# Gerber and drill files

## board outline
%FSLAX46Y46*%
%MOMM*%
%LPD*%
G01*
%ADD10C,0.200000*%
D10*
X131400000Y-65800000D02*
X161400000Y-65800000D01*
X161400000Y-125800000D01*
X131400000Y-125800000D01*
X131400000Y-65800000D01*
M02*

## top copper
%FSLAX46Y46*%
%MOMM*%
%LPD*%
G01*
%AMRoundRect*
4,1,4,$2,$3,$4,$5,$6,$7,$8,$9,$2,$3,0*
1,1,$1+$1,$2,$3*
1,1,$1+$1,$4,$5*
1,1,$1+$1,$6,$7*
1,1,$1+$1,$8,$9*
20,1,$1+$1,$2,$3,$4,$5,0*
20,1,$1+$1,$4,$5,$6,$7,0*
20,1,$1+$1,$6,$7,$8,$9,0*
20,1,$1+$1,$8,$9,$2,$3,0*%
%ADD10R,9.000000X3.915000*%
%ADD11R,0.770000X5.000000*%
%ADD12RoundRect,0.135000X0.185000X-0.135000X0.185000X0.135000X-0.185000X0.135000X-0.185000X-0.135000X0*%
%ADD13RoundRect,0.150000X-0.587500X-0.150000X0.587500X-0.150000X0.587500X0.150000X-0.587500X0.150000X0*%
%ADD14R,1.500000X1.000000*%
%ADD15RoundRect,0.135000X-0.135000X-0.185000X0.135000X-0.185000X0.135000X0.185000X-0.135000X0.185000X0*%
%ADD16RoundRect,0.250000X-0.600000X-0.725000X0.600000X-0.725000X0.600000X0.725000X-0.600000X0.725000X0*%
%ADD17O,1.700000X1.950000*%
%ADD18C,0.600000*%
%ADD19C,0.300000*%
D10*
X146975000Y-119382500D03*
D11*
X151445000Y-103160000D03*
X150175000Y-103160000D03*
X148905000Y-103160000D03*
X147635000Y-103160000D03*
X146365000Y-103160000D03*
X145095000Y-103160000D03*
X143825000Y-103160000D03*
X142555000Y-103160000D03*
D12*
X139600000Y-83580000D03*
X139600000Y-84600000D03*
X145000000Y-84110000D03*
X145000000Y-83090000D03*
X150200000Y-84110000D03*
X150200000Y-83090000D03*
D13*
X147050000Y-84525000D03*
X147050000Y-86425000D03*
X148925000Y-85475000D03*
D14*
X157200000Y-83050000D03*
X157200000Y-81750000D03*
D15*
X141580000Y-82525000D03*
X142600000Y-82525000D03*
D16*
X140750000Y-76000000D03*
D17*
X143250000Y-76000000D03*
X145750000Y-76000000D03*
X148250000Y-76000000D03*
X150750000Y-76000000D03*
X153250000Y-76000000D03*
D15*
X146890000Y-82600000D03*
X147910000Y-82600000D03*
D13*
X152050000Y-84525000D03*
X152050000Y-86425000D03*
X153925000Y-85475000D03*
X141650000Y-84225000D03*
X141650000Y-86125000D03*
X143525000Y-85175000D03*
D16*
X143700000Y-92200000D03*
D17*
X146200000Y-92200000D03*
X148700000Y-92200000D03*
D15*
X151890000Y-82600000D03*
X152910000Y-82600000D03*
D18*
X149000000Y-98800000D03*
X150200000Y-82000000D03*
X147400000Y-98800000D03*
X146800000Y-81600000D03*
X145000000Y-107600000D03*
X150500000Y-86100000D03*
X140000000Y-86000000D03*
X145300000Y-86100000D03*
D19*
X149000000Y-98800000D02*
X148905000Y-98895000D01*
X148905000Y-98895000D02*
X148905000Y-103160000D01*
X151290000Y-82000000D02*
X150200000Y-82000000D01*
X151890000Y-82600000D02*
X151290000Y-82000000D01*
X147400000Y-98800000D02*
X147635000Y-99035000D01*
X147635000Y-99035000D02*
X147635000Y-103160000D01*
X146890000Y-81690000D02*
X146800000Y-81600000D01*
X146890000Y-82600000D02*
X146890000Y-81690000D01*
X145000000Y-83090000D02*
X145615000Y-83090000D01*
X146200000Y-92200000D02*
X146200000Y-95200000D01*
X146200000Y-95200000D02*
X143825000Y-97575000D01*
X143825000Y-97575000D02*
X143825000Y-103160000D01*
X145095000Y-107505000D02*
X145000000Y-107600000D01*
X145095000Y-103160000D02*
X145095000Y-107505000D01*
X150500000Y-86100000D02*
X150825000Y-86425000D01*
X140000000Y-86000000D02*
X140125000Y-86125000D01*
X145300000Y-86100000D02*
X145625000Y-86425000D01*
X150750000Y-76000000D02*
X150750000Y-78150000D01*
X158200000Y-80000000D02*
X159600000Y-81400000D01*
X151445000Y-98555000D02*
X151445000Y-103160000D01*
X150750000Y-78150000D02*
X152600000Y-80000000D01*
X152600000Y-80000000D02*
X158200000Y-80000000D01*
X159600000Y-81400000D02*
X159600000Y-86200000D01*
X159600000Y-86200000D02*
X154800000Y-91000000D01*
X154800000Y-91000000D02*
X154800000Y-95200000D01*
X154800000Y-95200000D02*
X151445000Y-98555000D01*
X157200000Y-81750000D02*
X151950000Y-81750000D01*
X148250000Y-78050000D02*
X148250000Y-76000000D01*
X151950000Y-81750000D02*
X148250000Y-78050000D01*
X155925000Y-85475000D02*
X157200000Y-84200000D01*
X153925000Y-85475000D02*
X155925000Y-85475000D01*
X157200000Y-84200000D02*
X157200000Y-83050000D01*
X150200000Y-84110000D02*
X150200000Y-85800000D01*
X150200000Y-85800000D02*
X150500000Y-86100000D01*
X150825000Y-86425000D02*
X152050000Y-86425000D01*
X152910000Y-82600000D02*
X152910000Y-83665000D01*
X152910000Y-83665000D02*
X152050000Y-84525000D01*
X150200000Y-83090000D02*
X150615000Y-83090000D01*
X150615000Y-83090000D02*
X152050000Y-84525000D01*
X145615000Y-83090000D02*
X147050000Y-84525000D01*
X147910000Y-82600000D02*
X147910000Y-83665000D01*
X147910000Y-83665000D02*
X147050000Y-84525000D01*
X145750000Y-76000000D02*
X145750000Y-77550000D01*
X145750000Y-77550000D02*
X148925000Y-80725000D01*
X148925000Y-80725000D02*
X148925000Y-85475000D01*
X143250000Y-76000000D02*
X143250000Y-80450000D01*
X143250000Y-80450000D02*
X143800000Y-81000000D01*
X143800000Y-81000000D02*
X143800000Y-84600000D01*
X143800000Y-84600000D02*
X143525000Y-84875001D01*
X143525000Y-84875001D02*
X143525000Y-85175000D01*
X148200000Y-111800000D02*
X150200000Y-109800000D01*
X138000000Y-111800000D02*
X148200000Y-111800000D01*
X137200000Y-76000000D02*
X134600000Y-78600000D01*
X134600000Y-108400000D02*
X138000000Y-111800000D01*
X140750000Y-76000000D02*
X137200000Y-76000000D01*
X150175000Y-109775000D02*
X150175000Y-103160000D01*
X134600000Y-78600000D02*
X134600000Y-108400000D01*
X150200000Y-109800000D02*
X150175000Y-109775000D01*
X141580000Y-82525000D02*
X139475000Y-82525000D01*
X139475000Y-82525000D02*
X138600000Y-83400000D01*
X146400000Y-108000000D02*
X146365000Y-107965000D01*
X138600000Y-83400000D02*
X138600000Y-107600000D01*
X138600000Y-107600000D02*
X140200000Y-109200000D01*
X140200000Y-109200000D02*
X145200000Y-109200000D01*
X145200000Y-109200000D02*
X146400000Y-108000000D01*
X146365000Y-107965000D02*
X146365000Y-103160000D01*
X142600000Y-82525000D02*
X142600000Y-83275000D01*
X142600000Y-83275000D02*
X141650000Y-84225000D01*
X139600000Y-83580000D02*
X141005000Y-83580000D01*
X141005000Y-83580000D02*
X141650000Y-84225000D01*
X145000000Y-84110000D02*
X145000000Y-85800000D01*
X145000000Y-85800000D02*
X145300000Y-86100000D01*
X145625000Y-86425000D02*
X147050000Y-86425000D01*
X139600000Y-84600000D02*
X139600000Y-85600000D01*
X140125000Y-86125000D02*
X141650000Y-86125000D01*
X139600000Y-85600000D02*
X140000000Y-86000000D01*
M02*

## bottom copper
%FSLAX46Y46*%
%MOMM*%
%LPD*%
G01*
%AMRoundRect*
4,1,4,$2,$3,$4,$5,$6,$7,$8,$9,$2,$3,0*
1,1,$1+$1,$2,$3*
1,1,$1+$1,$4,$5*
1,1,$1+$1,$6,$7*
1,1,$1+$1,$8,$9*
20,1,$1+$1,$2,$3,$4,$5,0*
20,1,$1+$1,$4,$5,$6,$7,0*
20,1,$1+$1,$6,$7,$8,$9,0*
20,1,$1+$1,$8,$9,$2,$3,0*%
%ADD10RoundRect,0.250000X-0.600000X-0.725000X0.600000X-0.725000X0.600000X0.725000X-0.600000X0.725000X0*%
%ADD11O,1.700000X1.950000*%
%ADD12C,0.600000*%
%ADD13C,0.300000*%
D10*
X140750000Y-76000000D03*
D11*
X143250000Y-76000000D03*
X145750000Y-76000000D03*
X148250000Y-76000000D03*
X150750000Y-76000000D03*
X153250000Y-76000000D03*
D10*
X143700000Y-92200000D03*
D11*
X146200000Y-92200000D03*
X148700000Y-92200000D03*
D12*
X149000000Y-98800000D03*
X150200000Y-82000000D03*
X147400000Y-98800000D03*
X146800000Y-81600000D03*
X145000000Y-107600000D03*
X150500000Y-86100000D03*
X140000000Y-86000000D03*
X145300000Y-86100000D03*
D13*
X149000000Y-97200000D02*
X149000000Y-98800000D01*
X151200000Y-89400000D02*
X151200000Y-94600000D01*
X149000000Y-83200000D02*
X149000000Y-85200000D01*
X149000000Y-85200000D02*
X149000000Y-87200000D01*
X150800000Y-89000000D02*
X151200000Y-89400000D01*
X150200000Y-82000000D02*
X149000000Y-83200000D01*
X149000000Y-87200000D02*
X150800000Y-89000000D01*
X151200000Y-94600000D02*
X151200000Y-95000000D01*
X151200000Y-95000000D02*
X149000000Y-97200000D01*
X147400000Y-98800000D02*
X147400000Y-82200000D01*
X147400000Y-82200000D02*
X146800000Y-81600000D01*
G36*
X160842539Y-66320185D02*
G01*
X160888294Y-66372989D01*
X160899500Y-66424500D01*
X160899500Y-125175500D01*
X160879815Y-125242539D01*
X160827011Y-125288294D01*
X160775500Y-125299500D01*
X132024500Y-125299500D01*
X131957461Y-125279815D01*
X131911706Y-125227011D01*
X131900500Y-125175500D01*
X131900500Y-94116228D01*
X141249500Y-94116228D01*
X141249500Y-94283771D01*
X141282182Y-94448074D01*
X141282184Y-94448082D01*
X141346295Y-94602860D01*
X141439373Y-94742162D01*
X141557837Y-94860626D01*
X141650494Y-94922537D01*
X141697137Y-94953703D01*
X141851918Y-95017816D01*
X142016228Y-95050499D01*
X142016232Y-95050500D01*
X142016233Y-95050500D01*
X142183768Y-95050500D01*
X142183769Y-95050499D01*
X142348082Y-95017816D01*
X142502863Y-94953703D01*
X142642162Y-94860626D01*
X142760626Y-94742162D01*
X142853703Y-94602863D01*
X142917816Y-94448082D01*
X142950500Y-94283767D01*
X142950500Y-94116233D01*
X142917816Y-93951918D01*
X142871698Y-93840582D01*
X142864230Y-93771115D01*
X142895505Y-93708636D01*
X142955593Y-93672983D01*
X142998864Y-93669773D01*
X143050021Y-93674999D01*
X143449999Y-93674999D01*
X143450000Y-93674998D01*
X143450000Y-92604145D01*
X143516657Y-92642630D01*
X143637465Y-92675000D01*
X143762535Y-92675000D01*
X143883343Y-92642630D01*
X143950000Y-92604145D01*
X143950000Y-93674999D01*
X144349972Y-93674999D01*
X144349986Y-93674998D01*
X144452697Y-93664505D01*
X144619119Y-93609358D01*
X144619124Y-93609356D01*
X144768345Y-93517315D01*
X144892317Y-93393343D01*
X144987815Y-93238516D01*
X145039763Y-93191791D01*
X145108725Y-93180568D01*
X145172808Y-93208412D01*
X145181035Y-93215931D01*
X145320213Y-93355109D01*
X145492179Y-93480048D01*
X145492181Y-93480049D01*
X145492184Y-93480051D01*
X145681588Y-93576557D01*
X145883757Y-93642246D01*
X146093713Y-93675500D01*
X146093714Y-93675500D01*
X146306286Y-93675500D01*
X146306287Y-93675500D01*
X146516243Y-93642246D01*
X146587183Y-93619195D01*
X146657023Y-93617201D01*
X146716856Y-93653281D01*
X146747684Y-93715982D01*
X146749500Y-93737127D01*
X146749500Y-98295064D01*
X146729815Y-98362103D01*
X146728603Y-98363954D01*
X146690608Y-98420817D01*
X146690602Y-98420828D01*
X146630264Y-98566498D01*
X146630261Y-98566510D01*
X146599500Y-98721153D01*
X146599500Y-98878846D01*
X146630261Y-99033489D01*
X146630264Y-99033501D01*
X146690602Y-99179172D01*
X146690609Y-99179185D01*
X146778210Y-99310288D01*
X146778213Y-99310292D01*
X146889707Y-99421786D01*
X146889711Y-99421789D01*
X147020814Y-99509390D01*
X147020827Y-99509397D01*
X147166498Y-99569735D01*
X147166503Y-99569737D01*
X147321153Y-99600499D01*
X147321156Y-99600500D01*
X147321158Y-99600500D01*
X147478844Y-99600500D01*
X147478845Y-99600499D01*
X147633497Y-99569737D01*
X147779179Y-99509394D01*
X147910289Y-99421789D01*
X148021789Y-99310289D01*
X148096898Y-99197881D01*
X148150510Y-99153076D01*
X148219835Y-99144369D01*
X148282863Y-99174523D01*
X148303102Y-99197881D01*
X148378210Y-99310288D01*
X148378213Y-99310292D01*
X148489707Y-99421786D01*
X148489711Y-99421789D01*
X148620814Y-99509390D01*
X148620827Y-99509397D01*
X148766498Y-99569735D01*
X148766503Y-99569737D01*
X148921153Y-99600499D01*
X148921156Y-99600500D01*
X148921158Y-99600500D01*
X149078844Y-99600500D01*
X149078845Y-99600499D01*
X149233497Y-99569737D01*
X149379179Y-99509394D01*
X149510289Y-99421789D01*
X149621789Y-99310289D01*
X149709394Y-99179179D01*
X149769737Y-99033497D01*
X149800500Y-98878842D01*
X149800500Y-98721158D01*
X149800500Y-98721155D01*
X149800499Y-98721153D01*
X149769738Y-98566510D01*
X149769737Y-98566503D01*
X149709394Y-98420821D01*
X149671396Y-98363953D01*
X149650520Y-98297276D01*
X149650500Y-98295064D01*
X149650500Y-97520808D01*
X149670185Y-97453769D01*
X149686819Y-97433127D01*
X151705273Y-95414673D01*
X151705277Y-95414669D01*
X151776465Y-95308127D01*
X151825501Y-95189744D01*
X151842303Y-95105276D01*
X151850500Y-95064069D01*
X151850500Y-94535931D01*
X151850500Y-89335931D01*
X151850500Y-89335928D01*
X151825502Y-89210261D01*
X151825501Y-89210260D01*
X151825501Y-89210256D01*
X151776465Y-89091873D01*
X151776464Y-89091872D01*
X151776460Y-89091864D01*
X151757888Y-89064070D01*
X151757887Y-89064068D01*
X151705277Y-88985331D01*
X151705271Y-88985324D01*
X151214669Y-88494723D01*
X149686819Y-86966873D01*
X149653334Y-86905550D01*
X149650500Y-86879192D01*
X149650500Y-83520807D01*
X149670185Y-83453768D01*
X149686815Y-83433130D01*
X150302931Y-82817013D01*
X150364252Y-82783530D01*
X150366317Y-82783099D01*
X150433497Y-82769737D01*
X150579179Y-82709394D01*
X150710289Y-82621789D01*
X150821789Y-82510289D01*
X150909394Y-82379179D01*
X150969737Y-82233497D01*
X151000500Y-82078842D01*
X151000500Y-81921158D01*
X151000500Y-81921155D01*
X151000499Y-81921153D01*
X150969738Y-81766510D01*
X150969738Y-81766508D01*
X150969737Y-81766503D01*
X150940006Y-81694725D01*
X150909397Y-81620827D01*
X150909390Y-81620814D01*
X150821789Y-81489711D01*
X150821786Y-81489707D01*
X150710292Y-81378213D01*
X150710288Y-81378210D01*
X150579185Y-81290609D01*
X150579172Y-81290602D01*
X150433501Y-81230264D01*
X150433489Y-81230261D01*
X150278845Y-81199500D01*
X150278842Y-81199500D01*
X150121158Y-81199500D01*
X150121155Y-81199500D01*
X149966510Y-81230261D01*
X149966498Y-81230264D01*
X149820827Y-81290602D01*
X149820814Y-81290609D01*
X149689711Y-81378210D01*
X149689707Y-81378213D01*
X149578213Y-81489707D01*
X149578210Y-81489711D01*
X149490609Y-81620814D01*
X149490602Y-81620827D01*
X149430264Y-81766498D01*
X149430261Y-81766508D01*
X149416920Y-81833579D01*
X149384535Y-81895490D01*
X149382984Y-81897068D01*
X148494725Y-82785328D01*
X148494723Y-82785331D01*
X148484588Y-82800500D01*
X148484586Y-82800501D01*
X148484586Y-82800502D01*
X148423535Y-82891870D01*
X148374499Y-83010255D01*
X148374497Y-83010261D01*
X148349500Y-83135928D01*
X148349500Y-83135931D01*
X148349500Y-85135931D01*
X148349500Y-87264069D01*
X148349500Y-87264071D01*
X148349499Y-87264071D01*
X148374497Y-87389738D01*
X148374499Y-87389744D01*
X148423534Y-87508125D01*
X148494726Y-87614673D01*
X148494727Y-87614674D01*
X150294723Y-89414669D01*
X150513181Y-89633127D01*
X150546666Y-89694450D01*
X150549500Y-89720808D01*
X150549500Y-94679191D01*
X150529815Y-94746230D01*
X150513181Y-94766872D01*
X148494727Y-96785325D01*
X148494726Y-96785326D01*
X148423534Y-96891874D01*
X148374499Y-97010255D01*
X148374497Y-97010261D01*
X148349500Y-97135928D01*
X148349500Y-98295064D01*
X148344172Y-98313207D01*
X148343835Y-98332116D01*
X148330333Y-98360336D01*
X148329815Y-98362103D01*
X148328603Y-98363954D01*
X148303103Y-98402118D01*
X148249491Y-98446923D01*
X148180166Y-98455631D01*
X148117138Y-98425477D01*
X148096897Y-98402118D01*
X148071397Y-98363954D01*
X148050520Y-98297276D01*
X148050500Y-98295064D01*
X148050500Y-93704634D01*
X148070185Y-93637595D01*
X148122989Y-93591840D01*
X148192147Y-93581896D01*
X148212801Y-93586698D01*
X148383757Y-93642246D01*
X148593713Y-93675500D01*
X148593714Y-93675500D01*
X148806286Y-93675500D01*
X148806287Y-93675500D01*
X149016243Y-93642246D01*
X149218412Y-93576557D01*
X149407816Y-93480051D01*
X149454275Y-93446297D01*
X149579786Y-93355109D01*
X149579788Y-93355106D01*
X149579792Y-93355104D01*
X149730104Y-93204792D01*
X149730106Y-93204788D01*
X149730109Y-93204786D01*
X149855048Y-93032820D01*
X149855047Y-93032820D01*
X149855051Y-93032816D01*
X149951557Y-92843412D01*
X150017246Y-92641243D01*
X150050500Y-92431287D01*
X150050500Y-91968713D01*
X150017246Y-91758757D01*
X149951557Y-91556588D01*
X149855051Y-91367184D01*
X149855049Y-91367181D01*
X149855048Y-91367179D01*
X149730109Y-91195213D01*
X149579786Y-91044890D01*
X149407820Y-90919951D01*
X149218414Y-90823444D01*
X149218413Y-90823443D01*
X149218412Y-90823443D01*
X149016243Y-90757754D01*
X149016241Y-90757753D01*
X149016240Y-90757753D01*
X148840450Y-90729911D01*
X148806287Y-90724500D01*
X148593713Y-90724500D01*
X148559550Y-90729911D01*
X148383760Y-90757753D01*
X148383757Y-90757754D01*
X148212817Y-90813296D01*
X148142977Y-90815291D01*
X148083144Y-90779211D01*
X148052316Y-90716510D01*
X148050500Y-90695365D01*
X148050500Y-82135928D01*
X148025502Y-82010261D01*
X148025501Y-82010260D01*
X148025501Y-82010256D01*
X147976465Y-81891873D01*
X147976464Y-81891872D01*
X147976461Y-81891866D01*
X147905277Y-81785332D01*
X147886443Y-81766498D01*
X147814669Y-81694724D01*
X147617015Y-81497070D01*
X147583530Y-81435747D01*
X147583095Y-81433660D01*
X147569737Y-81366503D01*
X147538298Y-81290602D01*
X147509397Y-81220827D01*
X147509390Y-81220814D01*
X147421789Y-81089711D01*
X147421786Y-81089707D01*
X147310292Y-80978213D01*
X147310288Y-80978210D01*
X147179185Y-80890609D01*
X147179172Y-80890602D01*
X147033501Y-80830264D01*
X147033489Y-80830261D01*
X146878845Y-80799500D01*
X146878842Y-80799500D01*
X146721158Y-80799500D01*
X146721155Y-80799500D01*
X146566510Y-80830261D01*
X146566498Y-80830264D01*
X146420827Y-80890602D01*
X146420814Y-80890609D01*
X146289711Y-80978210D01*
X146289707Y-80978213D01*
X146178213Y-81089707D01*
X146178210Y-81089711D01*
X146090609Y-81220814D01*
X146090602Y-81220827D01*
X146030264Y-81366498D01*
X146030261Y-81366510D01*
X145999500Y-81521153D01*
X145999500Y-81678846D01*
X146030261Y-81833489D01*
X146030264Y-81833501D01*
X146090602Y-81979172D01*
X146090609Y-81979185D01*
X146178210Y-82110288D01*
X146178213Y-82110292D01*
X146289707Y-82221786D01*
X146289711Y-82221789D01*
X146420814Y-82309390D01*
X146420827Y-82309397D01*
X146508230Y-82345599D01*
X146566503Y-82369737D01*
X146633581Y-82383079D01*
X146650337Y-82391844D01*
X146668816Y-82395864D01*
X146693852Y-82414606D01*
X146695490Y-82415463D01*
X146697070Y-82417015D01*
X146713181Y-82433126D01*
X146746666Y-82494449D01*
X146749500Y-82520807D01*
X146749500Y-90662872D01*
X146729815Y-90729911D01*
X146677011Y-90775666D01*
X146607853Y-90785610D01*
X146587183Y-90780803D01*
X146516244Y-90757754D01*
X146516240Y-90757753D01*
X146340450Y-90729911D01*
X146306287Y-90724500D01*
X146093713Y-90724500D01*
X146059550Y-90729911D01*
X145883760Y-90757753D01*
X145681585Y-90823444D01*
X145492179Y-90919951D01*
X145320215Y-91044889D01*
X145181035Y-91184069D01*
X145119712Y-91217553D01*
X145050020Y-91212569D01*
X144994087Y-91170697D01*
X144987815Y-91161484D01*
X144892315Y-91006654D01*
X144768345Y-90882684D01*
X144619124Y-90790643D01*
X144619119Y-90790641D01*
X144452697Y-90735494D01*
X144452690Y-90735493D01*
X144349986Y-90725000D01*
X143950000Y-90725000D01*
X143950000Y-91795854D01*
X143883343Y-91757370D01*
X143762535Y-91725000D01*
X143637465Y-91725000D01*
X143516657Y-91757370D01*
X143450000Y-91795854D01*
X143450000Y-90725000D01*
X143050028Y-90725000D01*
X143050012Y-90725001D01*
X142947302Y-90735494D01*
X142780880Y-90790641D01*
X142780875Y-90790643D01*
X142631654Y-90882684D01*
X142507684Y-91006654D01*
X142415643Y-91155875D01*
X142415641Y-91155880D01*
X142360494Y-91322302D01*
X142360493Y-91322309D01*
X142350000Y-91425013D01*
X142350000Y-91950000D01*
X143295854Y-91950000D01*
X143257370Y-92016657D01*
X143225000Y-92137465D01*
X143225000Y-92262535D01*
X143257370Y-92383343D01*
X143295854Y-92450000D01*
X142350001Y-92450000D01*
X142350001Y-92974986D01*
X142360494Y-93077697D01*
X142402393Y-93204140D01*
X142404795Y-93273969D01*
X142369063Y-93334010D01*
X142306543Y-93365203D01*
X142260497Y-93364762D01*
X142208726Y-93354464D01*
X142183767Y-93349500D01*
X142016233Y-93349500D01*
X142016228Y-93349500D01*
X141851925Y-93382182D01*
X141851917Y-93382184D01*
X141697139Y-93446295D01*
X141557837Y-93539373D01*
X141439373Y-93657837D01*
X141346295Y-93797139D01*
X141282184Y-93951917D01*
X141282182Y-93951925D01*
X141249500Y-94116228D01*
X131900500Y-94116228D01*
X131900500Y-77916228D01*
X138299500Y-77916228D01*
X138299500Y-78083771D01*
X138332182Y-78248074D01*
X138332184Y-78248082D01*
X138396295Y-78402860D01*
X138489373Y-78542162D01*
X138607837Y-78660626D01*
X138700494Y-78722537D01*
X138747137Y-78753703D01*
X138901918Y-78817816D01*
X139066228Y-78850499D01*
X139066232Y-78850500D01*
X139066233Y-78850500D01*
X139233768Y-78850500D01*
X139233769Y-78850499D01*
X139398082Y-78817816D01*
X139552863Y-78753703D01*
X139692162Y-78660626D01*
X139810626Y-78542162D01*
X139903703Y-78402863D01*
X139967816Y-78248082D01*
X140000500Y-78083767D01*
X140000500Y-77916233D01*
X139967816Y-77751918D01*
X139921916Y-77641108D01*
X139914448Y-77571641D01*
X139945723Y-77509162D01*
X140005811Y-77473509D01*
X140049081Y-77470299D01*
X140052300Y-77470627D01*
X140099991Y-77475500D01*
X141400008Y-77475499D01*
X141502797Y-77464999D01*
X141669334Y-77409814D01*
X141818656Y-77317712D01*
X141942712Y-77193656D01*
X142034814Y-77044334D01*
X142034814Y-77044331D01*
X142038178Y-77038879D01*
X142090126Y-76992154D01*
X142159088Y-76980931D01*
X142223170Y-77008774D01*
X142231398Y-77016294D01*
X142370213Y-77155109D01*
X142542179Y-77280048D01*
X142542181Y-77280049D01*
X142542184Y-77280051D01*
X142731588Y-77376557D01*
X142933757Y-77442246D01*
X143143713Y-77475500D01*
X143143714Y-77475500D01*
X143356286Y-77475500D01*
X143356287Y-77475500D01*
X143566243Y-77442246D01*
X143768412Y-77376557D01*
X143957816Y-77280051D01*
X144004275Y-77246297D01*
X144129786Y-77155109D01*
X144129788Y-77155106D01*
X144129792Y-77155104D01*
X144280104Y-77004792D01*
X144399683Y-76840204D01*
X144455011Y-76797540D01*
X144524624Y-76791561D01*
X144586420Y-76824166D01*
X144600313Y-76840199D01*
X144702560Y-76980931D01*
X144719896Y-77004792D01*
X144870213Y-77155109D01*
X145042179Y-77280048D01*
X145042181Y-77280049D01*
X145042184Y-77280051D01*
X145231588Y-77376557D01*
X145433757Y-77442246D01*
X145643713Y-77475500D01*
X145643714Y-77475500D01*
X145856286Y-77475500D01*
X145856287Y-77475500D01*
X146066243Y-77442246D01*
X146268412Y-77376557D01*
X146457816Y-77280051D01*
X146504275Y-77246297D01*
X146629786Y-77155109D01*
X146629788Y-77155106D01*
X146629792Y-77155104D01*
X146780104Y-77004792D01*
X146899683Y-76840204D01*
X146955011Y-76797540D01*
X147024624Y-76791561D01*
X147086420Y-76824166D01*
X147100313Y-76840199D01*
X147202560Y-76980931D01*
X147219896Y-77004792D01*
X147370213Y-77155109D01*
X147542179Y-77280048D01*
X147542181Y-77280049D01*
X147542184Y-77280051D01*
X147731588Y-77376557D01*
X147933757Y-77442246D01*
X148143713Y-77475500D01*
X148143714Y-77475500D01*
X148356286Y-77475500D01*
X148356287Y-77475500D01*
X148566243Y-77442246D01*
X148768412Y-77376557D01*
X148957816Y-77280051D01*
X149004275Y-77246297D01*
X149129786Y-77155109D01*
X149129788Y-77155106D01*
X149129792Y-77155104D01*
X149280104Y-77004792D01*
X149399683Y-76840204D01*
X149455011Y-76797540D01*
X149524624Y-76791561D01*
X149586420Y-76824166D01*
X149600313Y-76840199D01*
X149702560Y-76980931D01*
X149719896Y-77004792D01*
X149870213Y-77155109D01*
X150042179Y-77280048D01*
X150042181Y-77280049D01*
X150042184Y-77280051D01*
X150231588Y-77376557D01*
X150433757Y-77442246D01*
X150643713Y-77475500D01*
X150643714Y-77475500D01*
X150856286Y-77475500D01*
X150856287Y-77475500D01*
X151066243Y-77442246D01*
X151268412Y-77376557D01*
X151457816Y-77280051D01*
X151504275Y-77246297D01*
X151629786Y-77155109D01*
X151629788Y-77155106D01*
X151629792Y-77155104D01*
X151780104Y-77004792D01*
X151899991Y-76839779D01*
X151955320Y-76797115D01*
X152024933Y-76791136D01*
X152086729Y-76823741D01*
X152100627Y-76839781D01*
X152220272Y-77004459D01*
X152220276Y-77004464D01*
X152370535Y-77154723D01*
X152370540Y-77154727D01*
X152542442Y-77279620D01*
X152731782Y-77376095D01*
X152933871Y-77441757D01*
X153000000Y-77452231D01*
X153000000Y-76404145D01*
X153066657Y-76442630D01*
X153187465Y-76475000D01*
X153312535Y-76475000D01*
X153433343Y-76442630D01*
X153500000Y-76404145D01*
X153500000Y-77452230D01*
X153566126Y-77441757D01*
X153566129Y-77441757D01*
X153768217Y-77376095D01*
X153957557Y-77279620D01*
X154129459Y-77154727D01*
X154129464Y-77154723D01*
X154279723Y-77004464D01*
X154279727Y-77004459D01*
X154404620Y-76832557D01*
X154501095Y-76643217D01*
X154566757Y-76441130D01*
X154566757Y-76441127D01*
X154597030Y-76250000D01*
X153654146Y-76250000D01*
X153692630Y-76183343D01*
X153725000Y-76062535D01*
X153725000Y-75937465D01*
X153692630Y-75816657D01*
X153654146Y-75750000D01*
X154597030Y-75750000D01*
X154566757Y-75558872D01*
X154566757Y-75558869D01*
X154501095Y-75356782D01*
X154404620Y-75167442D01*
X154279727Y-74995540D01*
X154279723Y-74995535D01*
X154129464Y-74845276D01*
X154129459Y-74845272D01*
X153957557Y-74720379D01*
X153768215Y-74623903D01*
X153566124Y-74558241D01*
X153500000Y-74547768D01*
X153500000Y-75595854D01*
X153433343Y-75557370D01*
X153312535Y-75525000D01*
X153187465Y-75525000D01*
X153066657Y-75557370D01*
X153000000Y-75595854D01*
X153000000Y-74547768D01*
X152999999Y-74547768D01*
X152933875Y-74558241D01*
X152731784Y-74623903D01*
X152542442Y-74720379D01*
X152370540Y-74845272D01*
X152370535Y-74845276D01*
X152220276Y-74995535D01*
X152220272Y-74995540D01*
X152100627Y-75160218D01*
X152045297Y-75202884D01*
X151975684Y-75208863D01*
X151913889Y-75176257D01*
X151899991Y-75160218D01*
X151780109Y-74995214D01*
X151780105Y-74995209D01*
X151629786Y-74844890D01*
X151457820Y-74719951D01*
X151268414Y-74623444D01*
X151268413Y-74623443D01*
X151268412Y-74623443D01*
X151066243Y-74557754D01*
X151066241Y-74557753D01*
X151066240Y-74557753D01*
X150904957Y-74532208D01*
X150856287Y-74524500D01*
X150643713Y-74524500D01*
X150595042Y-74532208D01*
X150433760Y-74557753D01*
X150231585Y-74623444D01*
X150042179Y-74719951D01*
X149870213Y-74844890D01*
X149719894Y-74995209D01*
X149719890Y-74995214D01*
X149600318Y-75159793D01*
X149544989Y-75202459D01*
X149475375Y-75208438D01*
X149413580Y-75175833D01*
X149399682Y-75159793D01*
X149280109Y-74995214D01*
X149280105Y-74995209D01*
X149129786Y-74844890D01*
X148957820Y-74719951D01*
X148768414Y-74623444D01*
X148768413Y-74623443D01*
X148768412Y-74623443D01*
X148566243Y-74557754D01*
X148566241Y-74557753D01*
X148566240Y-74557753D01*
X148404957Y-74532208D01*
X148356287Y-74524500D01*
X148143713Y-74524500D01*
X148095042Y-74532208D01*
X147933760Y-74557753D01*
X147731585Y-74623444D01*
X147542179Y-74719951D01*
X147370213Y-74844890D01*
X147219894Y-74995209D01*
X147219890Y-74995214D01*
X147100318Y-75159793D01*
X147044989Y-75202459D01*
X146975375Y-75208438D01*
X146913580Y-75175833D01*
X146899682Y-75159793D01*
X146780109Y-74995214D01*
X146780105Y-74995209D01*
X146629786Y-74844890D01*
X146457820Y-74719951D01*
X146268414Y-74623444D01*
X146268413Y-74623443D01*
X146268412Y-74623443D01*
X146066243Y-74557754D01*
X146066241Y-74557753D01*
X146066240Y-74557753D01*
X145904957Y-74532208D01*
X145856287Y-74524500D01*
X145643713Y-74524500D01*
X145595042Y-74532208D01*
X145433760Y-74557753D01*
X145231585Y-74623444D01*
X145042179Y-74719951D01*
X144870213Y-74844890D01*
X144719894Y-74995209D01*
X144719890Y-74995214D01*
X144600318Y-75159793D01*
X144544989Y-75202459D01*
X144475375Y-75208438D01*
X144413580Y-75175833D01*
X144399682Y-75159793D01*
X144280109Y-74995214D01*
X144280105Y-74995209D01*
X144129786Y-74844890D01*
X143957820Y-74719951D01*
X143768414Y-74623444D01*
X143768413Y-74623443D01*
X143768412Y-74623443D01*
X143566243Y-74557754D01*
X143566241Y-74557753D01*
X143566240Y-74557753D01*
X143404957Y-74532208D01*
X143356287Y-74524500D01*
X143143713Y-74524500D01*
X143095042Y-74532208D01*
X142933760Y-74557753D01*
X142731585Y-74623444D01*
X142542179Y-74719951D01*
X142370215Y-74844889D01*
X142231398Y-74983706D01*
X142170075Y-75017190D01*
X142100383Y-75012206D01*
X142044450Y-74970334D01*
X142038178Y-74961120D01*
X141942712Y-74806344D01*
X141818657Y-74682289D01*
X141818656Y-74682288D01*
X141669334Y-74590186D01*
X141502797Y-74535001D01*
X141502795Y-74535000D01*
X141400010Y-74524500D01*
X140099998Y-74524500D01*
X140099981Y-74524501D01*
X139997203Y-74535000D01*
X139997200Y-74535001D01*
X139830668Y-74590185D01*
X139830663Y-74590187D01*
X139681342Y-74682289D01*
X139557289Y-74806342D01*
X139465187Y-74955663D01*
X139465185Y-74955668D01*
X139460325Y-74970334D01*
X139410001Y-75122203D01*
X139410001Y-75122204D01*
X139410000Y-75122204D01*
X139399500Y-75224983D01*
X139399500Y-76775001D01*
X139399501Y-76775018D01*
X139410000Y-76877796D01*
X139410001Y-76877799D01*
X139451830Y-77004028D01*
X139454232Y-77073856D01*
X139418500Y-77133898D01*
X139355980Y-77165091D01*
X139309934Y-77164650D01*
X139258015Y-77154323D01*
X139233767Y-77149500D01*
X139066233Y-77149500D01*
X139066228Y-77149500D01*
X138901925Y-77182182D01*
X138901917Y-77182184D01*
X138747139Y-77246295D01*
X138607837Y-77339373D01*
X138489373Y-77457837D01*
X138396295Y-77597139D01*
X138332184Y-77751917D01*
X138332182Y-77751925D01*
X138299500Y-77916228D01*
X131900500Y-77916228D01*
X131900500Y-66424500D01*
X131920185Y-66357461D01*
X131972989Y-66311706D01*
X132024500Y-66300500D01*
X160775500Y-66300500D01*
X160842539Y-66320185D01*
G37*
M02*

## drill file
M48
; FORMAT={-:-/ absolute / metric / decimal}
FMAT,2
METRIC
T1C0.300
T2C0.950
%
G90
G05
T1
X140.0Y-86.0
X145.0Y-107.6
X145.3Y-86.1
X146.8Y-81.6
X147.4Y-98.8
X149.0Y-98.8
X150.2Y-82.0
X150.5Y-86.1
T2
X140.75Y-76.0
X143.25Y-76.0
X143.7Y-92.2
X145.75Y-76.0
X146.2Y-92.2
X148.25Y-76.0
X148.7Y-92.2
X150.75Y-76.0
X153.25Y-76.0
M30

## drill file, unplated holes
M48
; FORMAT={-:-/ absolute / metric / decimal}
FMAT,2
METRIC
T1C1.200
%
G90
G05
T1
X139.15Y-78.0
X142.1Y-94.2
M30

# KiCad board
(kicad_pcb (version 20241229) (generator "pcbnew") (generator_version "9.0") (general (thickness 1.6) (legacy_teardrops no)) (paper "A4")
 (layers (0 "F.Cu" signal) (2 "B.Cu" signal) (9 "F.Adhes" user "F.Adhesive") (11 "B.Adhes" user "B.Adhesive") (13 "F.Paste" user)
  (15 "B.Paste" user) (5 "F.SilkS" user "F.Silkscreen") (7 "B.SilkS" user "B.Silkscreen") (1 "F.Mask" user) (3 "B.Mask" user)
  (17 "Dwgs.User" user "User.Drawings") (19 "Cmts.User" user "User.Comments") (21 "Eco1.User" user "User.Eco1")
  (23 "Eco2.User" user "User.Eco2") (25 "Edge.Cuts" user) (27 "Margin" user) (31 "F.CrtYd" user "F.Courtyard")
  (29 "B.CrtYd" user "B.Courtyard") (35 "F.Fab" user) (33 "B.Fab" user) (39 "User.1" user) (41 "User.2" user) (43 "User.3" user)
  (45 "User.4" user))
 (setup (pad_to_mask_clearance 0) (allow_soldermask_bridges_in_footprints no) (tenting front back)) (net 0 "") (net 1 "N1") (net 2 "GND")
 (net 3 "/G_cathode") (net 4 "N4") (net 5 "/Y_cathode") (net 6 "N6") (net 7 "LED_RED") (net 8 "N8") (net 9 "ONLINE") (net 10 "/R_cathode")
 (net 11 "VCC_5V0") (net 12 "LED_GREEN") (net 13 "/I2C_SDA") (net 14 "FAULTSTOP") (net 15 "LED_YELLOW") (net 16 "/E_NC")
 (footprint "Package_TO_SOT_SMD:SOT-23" (layer "F.Cu") (at 147.9875 85.475)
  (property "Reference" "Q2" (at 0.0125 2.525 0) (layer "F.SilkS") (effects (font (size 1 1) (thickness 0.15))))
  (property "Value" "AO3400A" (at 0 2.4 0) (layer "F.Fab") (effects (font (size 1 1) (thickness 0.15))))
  (pad "1" smd roundrect (at -0.9375 -0.95) (size 1.475 0.6) (layers "F.Cu" "F.Mask" "F.Paste") (roundrect_rratio 0.25) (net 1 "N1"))
  (pad "2" smd roundrect (at -0.9375 0.95) (size 1.475 0.6) (layers "F.Cu" "F.Mask" "F.Paste") (roundrect_rratio 0.25) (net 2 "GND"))
  (pad "3" smd roundrect (at 0.9375 0) (size 1.475 0.6) (layers "F.Cu" "F.Mask" "F.Paste") (roundrect_rratio 0.25) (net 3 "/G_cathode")))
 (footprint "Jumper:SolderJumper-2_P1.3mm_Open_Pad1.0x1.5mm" (layer "F.Cu") (at 157.2 82.4 90)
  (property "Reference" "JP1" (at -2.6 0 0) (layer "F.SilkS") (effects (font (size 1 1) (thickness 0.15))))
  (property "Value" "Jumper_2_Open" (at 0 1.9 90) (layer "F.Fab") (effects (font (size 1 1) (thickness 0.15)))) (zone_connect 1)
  (pad "1" smd rect (at -0.65 0 90) (size 1 1.5) (layers "F.Cu" "F.Mask") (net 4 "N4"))
  (pad "2" smd rect (at 0.65 0 90) (size 1 1.5) (layers "F.Cu" "F.Mask") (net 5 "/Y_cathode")))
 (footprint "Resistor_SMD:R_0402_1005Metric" (layer "F.Cu") (at 145 83.6 90)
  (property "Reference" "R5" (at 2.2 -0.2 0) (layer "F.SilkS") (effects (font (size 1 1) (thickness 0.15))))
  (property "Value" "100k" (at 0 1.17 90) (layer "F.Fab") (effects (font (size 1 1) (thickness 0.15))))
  (pad "1" smd roundrect (at -0.51 0 90) (size 0.54 0.64) (layers "F.Cu" "F.Mask" "F.Paste") (roundrect_rratio 0.25) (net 2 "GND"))
  (pad "2" smd roundrect (at 0.51 0 90) (size 0.54 0.64) (layers "F.Cu" "F.Mask" "F.Paste") (roundrect_rratio 0.25) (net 1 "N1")))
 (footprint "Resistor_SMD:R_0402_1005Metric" (layer "F.Cu") (at 150.2 83.6 90)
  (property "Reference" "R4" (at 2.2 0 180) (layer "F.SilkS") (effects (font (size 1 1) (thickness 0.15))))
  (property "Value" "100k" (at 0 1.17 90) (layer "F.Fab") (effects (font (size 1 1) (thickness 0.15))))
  (pad "1" smd roundrect (at -0.51 0 90) (size 0.54 0.64) (layers "F.Cu" "F.Mask" "F.Paste") (roundrect_rratio 0.25) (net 2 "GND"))
  (pad "2" smd roundrect (at 0.51 0 90) (size 0.54 0.64) (layers "F.Cu" "F.Mask" "F.Paste") (roundrect_rratio 0.25) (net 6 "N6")))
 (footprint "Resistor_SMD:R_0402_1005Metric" (layer "F.Cu") (at 142.09 82.525)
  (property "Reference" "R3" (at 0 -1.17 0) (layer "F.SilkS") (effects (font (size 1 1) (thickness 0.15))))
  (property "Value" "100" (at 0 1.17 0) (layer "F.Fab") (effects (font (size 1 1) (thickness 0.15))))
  (pad "1" smd roundrect (at -0.51 0) (size 0.54 0.64) (layers "F.Cu" "F.Mask" "F.Paste") (roundrect_rratio 0.25) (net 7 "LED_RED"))
  (pad "2" smd roundrect (at 0.51 0) (size 0.54 0.64) (layers "F.Cu" "F.Mask" "F.Paste") (roundrect_rratio 0.25) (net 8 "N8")))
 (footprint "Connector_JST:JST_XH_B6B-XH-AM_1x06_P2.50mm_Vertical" (layer "F.Cu") (at 140.75 76)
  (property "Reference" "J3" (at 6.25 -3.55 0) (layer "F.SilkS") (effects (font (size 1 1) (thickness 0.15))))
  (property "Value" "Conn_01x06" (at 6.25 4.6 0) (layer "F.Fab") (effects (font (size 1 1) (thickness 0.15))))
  (pad "" np_thru_hole circle (at -1.6 2) (size 1.2 1.2) (drill 1.2) (layers "*.Cu" "*.Mask"))
  (pad "1" thru_hole roundrect (at 0 0) (size 1.7 1.95) (drill 0.95) (layers "*.Cu" "*.Mask") (remove_unused_layers no)
   (roundrect_rratio 0.147059) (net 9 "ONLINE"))
  (pad "2" thru_hole oval (at 2.5 0) (size 1.7 1.95) (drill 0.95) (layers "*.Cu" "*.Mask") (remove_unused_layers no) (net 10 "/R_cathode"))
  (pad "3" thru_hole oval (at 5 0) (size 1.7 1.95) (drill 0.95) (layers "*.Cu" "*.Mask") (remove_unused_layers no) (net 3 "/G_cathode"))
  (pad "4" thru_hole oval (at 7.5 0) (size 1.7 1.95) (drill 0.95) (layers "*.Cu" "*.Mask") (remove_unused_layers no) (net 5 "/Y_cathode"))
  (pad "5" thru_hole oval (at 10 0) (size 1.7 1.95) (drill 0.95) (layers "*.Cu" "*.Mask") (remove_unused_layers no) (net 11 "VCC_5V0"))
  (pad "6" thru_hole oval (at 12.5 0) (size 1.7 1.95) (drill 0.95) (layers "*.Cu" "*.Mask") (remove_unused_layers no) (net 2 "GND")))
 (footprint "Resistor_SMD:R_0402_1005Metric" (layer "F.Cu") (at 147.4 82.6)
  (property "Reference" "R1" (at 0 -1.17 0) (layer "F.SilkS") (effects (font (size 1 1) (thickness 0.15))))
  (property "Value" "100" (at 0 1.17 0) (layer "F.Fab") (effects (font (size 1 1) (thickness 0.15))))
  (pad "1" smd roundrect (at -0.51 0) (size 0.54 0.64) (layers "F.Cu" "F.Mask" "F.Paste") (roundrect_rratio 0.25) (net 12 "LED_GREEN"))
  (pad "2" smd roundrect (at 0.51 0) (size 0.54 0.64) (layers "F.Cu" "F.Mask" "F.Paste") (roundrect_rratio 0.25) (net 1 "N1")))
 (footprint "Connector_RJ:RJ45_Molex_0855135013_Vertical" (layer "F.Cu") (at 147 111)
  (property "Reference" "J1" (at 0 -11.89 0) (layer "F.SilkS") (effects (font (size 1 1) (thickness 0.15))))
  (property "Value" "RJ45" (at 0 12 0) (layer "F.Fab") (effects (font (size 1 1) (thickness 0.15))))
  (pad "1" smd rect (at -4.445 -7.84 180) (size 0.77 5) (layers "F.Cu" "F.Mask" "F.Paste") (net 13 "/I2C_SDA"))
  (pad "2" smd rect (at -3.175 -7.84 180) (size 0.77 5) (layers "F.Cu" "F.Mask" "F.Paste") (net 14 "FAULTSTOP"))
  (pad "3" smd rect (at -1.905 -7.84 180) (size 0.77 5) (layers "F.Cu" "F.Mask" "F.Paste") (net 2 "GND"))
  (pad "4" smd rect (at -0.635 -7.84 180) (size 0.77 5) (layers "F.Cu" "F.Mask" "F.Paste") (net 7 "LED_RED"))
  (pad "5" smd rect (at 0.635 -7.84 180) (size 0.77 5) (layers "F.Cu" "F.Mask" "F.Paste") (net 12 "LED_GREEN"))
  (pad "6" smd rect (at 1.905 -7.84 180) (size 0.77 5) (layers "F.Cu" "F.Mask" "F.Paste") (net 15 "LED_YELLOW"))
  (pad "7" smd rect (at 3.175 -7.84 180) (size 0.77 5) (layers "F.Cu" "F.Mask" "F.Paste") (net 9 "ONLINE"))
  (pad "8" smd rect (at 4.445 -7.84 180) (size 0.77 5) (layers "F.Cu" "F.Mask" "F.Paste") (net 11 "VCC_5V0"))
  (pad "L" smd rect (at -0.025 8.3825 180) (size 9 3.915) (layers "F.Cu" "F.Mask" "F.Paste")))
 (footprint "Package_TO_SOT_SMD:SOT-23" (layer "F.Cu") (at 152.9875 85.475)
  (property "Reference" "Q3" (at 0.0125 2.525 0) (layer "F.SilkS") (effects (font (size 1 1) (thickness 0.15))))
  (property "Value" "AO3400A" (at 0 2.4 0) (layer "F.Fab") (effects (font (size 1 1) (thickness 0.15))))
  (pad "1" smd roundrect (at -0.9375 -0.95) (size 1.475 0.6) (layers "F.Cu" "F.Mask" "F.Paste") (roundrect_rratio 0.25) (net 6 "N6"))
  (pad "2" smd roundrect (at -0.9375 0.95) (size 1.475 0.6) (layers "F.Cu" "F.Mask" "F.Paste") (roundrect_rratio 0.25) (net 2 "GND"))
  (pad "3" smd roundrect (at 0.9375 0) (size 1.475 0.6) (layers "F.Cu" "F.Mask" "F.Paste") (roundrect_rratio 0.25) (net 4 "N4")))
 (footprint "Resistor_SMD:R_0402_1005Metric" (layer "F.Cu") (at 139.6 84.09 90)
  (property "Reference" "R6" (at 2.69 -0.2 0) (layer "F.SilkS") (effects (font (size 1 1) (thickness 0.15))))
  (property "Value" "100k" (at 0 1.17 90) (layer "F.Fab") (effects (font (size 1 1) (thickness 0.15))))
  (pad "1" smd roundrect (at -0.51 0 90) (size 0.54 0.64) (layers "F.Cu" "F.Mask" "F.Paste") (roundrect_rratio 0.25) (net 2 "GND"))
  (pad "2" smd roundrect (at 0.51 0 90) (size 0.54 0.64) (layers "F.Cu" "F.Mask" "F.Paste") (roundrect_rratio 0.25) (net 8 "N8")))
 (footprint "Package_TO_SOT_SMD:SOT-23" (layer "F.Cu") (at 142.5875 85.175)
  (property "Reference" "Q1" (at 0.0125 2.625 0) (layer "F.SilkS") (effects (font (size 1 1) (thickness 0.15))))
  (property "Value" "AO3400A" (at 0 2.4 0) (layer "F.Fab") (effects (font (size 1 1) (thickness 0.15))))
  (pad "1" smd roundrect (at -0.9375 -0.95) (size 1.475 0.6) (layers "F.Cu" "F.Mask" "F.Paste") (roundrect_rratio 0.25) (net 8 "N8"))
  (pad "2" smd roundrect (at -0.9375 0.95) (size 1.475 0.6) (layers "F.Cu" "F.Mask" "F.Paste") (roundrect_rratio 0.25) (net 2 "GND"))
  (pad "3" smd roundrect (at 0.9375 0) (size 1.475 0.6) (layers "F.Cu" "F.Mask" "F.Paste") (roundrect_rratio 0.25) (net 10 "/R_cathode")))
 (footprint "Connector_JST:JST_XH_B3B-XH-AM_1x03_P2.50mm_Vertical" (layer "F.Cu") (at 143.7 92.2)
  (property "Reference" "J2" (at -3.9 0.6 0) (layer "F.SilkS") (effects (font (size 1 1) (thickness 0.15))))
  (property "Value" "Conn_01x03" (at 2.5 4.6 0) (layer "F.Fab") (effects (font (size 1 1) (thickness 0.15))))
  (pad "" np_thru_hole circle (at -1.6 2) (size 1.2 1.2) (drill 1.2) (layers "*.Cu" "*.Mask"))
  (pad "1" thru_hole roundrect (at 0 0) (size 1.7 1.95) (drill 0.95) (layers "*.Cu" "*.Mask") (remove_unused_layers no)
   (roundrect_rratio 0.147059) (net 2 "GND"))
  (pad "2" thru_hole oval (at 2.5 0) (size 1.7 1.95) (drill 0.95) (layers "*.Cu" "*.Mask") (remove_unused_layers no) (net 14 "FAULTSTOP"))
  (pad "3" thru_hole oval (at 5 0) (size 1.7 1.95) (drill 0.95) (layers "*.Cu" "*.Mask") (remove_unused_layers no) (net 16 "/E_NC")))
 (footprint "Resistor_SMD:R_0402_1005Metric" (layer "F.Cu") (at 152.4 82.6)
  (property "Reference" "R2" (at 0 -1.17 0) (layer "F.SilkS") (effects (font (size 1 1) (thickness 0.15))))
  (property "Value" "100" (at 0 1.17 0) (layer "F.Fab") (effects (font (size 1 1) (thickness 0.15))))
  (pad "1" smd roundrect (at -0.51 0) (size 0.54 0.64) (layers "F.Cu" "F.Mask" "F.Paste") (roundrect_rratio 0.25) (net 15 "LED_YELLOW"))
  (pad "2" smd roundrect (at 0.51 0) (size 0.54 0.64) (layers "F.Cu" "F.Mask" "F.Paste") (roundrect_rratio 0.25) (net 6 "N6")))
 (gr_rect (start 131.4 65.8) (end 161.4 125.8) (stroke (width 0.2) (type solid)) (fill no) (layer "Edge.Cuts"))
 (segment (start 146.2 95.2) (end 143.825 97.575) (width 0.3) (layer "F.Cu") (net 14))
 (segment (start 143.825 97.575) (end 143.825 103.16) (width 0.3) (layer "F.Cu") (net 14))
 (segment (start 146.2 92.2) (end 146.2 95.2) (width 0.3) (layer "F.Cu") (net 14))
 (segment (start 145.3 86.1) (end 145.625 86.425) (width 0.3) (layer "F.Cu") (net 2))
 (segment (start 145.625 86.425) (end 147.05 86.425) (width 0.3) (layer "F.Cu") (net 2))
 (segment (start 150.2 85.8) (end 150.5 86.1) (width 0.3) (layer "F.Cu") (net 2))
 (segment (start 140 86) (end 140.125 86.125) (width 0.3) (layer "F.Cu") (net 2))
 (segment (start 140.125 86.125) (end 141.65 86.125) (width 0.3) (layer "F.Cu") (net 2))
 (segment (start 150.825 86.425) (end 152.05 86.425) (width 0.3) (layer "F.Cu") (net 2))
 (segment (start 145 84.11) (end 145 85.8) (width 0.3) (layer "F.Cu") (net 2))
 (segment (start 139.6 84.6) (end 139.6 85.6) (width 0.3) (layer "F.Cu") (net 2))
 (segment (start 145.095 103.16) (end 145.095 107.505) (width 0.3) (layer "F.Cu") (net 2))
 (segment (start 145.095 107.505) (end 145 107.6) (width 0.3) (layer "F.Cu") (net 2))
 (segment (start 150.2 84.11) (end 150.2 85.8) (width 0.3) (layer "F.Cu") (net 2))
 (segment (start 150.5 86.1) (end 150.825 86.425) (width 0.3) (layer "F.Cu") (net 2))
 (segment (start 145 85.8) (end 145.3 86.1) (width 0.3) (layer "F.Cu") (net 2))
 (segment (start 139.6 85.6) (end 140 86) (width 0.3) (layer "F.Cu") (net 2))
 (via (at 145 107.6) (size 0.6) (drill 0.3) (layers "F.Cu" "B.Cu") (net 2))
 (via (at 140 86) (size 0.6) (drill 0.3) (layers "F.Cu" "B.Cu") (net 2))
 (via (at 145.3 86.1) (size 0.6) (drill 0.3) (layers "F.Cu" "B.Cu") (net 2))
 (via (at 150.5 86.1) (size 0.6) (drill 0.3) (layers "F.Cu" "B.Cu") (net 2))
 (segment (start 150.175 109.775) (end 150.175 103.16) (width 0.3) (layer "F.Cu") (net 9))
 (segment (start 140.75 76) (end 137.2 76) (width 0.3) (layer "F.Cu") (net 9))
 (segment (start 134.6 78.6) (end 134.6 108.4) (width 0.3) (layer "F.Cu") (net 9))
 (segment (start 148.2 111.8) (end 150.2 109.8) (width 0.3) (layer "F.Cu") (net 9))
 (segment (start 137.2 76) (end 134.6 78.6) (width 0.3) (layer "F.Cu") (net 9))
 (segment (start 150.2 109.8) (end 150.175 109.775) (width 0.3) (layer "F.Cu") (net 9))
 (segment (start 134.6 108.4) (end 138 111.8) (width 0.3) (layer "F.Cu") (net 9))
 (segment (start 138 111.8) (end 148.2 111.8) (width 0.3) (layer "F.Cu") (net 9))
 (segment (start 141.58 82.525) (end 139.475 82.525) (width 0.3) (layer "F.Cu") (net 7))
 (segment (start 139.475 82.525) (end 138.6 83.4) (width 0.3) (layer "F.Cu") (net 7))
 (segment (start 145.2 109.2) (end 146.4 108) (width 0.3) (layer "F.Cu") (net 7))
 (segment (start 140.2 109.2) (end 145.2 109.2) (width 0.3) (layer "F.Cu") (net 7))
 (segment (start 146.4 108) (end 146.365 107.965) (width 0.3) (layer "F.Cu") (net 7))
 (segment (start 138.6 107.6) (end 140.2 109.2) (width 0.3) (layer "F.Cu") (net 7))
 (segment (start 138.6 83.4) (end 138.6 107.6) (width 0.3) (layer "F.Cu") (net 7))
 (segment (start 146.365 107.965) (end 146.365 103.16) (width 0.3) (layer "F.Cu") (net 7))
 (segment (start 146.89 81.69) (end 146.8 81.6) (width 0.3) (layer "F.Cu") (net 12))
 (segment (start 147.635 99.035) (end 147.635 103.16) (width 0.3) (layer "F.Cu") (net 12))
 (segment (start 146.89 82.6) (end 146.89 81.69) (width 0.3) (layer "F.Cu") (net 12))
 (segment (start 147.4 98.8) (end 147.635 99.035) (width 0.3) (layer "F.Cu") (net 12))
 (via (at 147.4 98.8) (size 0.6) (drill 0.3) (layers "F.Cu" "B.Cu") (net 12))
 (via (at 146.8 81.6) (size 0.6) (drill 0.3) (layers "F.Cu" "B.Cu") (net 12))
 (segment (start 147.4 82.2) (end 146.8 81.6) (width 0.3) (layer "B.Cu") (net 12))
 (segment (start 147.4 98.8) (end 147.4 82.2) (width 0.3) (layer "B.Cu") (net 12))
 (segment (start 150.75 78.15) (end 152.6 80) (width 0.3) (layer "F.Cu") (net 11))
 (segment (start 150.75 76) (end 150.75 78.15) (width 0.3) (layer "F.Cu") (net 11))
 (segment (start 152.6 80) (end 158.2 80) (width 0.3) (layer "F.Cu") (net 11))
 (segment (start 151.445 98.555) (end 151.445 103.16) (width 0.3) (layer "F.Cu") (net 11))
 (segment (start 159.6 81.4) (end 159.6 86.2) (width 0.3) (layer "F.Cu") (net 11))
 (segment (start 154.8 91) (end 154.8 95.2) (width 0.3) (layer "F.Cu") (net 11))
 (segment (start 158.2 80) (end 159.6 81.4) (width 0.3) (layer "F.Cu") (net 11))
 (segment (start 154.8 95.2) (end 151.445 98.555) (width 0.3) (layer "F.Cu") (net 11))
 (segment (start 159.6 86.2) (end 154.8 91) (width 0.3) (layer "F.Cu") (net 11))
 (segment (start 151.89 82.6) (end 151.29 82) (width 0.3) (layer "F.Cu") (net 15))
 (segment (start 148.905 98.895) (end 148.905 103.16) (width 0.3) (layer "F.Cu") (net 15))
 (segment (start 151.29 82) (end 150.2 82) (width 0.3) (layer "F.Cu") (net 15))
 (segment (start 149 98.8) (end 148.905 98.895) (width 0.3) (layer "F.Cu") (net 15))
 (via (at 150.2 82) (size 0.6) (drill 0.3) (layers "F.Cu" "B.Cu") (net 15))
 (via (at 149 98.8) (size 0.6) (drill 0.3) (layers "F.Cu" "B.Cu") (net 15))
 (segment (start 151.2 95) (end 149 97.2) (width 0.3) (layer "B.Cu") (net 15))
 (segment (start 150.8 89) (end 151.2 89.4) (width 0.3) (layer "B.Cu") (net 15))
 (segment (start 151.2 94.6) (end 151.2 95) (width 0.3) (layer "B.Cu") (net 15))
 (segment (start 149 87.2) (end 150.8 89) (width 0.3) (layer "B.Cu") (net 15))
 (segment (start 149 97.2) (end 149 98.8) (width 0.3) (layer "B.Cu") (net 15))
 (segment (start 149 83.2) (end 149 85.2) (width 0.3) (layer "B.Cu") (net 15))
 (segment (start 150.2 82) (end 149 83.2) (width 0.3) (layer "B.Cu") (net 15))
 (segment (start 149 85.2) (end 149 87.2) (width 0.3) (layer "B.Cu") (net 15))
 (segment (start 151.2 89.4) (end 151.2 94.6) (width 0.3) (layer "B.Cu") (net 15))
 (segment (start 143.525 84.875001) (end 143.525 85.175) (width 0.3) (layer "F.Cu") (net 10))
 (segment (start 143.8 81) (end 143.8 84.6) (width 0.3) (layer "F.Cu") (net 10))
 (segment (start 143.25 76) (end 143.25 80.45) (width 0.3) (layer "F.Cu") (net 10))
 (segment (start 143.25 80.45) (end 143.8 81) (width 0.3) (layer "F.Cu") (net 10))
 (segment (start 143.8 84.6) (end 143.525 84.875001) (width 0.3) (layer "F.Cu") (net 10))
 (segment (start 145.75 76) (end 145.75 77.55) (width 0.3) (layer "F.Cu") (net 3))
 (segment (start 148.925 80.725) (end 148.925 85.475) (width 0.3) (layer "F.Cu") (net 3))
 (segment (start 145.75 77.55) (end 148.925 80.725) (width 0.3) (layer "F.Cu") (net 3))
 (segment (start 151.95 81.75) (end 148.25 78.05) (width 0.3) (layer "F.Cu") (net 5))
 (segment (start 157.2 81.75) (end 151.95 81.75) (width 0.3) (layer "F.Cu") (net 5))
 (segment (start 148.25 78.05) (end 148.25 76) (width 0.3) (layer "F.Cu") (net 5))
 (segment (start 153.925 85.475) (end 155.925 85.475) (width 0.3) (layer "F.Cu") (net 4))
 (segment (start 155.925 85.475) (end 157.2 84.2) (width 0.3) (layer "F.Cu") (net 4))
 (segment (start 157.2 84.2) (end 157.2 83.05) (width 0.3) (layer "F.Cu") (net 4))
 (segment (start 141.005 83.58) (end 141.65 84.225) (width 0.3) (layer "F.Cu") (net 8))
 (segment (start 142.6 83.275) (end 141.65 84.225) (width 0.3) (layer "F.Cu") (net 8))
 (segment (start 139.6 83.58) (end 141.005 83.58) (width 0.3) (layer "F.Cu") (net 8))
 (segment (start 142.6 82.525) (end 142.6 83.275) (width 0.3) (layer "F.Cu") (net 8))
 (segment (start 147.91 82.6) (end 147.91 83.665) (width 0.3) (layer "F.Cu") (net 1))
 (segment (start 147.91 83.665) (end 147.05 84.525) (width 0.3) (layer "F.Cu") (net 1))
 (segment (start 145.615 83.09) (end 147.05 84.525) (width 0.3) (layer "F.Cu") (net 1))
 (segment (start 145 83.09) (end 145.615 83.09) (width 0.3) (layer "F.Cu") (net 1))
 (segment (start 150.615 83.09) (end 152.05 84.525) (width 0.3) (layer "F.Cu") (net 6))
 (segment (start 150.2 83.09) (end 150.615 83.09) (width 0.3) (layer "F.Cu") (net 6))
 (segment (start 152.91 82.6) (end 152.91 83.665) (width 0.3) (layer "F.Cu") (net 6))
 (segment (start 152.91 83.665) (end 152.05 84.525) (width 0.3) (layer "F.Cu") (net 6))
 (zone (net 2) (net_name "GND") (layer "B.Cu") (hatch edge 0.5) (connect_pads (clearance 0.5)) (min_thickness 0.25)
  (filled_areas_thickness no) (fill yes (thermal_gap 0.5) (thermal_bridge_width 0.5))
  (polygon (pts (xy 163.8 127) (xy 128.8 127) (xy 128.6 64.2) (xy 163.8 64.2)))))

